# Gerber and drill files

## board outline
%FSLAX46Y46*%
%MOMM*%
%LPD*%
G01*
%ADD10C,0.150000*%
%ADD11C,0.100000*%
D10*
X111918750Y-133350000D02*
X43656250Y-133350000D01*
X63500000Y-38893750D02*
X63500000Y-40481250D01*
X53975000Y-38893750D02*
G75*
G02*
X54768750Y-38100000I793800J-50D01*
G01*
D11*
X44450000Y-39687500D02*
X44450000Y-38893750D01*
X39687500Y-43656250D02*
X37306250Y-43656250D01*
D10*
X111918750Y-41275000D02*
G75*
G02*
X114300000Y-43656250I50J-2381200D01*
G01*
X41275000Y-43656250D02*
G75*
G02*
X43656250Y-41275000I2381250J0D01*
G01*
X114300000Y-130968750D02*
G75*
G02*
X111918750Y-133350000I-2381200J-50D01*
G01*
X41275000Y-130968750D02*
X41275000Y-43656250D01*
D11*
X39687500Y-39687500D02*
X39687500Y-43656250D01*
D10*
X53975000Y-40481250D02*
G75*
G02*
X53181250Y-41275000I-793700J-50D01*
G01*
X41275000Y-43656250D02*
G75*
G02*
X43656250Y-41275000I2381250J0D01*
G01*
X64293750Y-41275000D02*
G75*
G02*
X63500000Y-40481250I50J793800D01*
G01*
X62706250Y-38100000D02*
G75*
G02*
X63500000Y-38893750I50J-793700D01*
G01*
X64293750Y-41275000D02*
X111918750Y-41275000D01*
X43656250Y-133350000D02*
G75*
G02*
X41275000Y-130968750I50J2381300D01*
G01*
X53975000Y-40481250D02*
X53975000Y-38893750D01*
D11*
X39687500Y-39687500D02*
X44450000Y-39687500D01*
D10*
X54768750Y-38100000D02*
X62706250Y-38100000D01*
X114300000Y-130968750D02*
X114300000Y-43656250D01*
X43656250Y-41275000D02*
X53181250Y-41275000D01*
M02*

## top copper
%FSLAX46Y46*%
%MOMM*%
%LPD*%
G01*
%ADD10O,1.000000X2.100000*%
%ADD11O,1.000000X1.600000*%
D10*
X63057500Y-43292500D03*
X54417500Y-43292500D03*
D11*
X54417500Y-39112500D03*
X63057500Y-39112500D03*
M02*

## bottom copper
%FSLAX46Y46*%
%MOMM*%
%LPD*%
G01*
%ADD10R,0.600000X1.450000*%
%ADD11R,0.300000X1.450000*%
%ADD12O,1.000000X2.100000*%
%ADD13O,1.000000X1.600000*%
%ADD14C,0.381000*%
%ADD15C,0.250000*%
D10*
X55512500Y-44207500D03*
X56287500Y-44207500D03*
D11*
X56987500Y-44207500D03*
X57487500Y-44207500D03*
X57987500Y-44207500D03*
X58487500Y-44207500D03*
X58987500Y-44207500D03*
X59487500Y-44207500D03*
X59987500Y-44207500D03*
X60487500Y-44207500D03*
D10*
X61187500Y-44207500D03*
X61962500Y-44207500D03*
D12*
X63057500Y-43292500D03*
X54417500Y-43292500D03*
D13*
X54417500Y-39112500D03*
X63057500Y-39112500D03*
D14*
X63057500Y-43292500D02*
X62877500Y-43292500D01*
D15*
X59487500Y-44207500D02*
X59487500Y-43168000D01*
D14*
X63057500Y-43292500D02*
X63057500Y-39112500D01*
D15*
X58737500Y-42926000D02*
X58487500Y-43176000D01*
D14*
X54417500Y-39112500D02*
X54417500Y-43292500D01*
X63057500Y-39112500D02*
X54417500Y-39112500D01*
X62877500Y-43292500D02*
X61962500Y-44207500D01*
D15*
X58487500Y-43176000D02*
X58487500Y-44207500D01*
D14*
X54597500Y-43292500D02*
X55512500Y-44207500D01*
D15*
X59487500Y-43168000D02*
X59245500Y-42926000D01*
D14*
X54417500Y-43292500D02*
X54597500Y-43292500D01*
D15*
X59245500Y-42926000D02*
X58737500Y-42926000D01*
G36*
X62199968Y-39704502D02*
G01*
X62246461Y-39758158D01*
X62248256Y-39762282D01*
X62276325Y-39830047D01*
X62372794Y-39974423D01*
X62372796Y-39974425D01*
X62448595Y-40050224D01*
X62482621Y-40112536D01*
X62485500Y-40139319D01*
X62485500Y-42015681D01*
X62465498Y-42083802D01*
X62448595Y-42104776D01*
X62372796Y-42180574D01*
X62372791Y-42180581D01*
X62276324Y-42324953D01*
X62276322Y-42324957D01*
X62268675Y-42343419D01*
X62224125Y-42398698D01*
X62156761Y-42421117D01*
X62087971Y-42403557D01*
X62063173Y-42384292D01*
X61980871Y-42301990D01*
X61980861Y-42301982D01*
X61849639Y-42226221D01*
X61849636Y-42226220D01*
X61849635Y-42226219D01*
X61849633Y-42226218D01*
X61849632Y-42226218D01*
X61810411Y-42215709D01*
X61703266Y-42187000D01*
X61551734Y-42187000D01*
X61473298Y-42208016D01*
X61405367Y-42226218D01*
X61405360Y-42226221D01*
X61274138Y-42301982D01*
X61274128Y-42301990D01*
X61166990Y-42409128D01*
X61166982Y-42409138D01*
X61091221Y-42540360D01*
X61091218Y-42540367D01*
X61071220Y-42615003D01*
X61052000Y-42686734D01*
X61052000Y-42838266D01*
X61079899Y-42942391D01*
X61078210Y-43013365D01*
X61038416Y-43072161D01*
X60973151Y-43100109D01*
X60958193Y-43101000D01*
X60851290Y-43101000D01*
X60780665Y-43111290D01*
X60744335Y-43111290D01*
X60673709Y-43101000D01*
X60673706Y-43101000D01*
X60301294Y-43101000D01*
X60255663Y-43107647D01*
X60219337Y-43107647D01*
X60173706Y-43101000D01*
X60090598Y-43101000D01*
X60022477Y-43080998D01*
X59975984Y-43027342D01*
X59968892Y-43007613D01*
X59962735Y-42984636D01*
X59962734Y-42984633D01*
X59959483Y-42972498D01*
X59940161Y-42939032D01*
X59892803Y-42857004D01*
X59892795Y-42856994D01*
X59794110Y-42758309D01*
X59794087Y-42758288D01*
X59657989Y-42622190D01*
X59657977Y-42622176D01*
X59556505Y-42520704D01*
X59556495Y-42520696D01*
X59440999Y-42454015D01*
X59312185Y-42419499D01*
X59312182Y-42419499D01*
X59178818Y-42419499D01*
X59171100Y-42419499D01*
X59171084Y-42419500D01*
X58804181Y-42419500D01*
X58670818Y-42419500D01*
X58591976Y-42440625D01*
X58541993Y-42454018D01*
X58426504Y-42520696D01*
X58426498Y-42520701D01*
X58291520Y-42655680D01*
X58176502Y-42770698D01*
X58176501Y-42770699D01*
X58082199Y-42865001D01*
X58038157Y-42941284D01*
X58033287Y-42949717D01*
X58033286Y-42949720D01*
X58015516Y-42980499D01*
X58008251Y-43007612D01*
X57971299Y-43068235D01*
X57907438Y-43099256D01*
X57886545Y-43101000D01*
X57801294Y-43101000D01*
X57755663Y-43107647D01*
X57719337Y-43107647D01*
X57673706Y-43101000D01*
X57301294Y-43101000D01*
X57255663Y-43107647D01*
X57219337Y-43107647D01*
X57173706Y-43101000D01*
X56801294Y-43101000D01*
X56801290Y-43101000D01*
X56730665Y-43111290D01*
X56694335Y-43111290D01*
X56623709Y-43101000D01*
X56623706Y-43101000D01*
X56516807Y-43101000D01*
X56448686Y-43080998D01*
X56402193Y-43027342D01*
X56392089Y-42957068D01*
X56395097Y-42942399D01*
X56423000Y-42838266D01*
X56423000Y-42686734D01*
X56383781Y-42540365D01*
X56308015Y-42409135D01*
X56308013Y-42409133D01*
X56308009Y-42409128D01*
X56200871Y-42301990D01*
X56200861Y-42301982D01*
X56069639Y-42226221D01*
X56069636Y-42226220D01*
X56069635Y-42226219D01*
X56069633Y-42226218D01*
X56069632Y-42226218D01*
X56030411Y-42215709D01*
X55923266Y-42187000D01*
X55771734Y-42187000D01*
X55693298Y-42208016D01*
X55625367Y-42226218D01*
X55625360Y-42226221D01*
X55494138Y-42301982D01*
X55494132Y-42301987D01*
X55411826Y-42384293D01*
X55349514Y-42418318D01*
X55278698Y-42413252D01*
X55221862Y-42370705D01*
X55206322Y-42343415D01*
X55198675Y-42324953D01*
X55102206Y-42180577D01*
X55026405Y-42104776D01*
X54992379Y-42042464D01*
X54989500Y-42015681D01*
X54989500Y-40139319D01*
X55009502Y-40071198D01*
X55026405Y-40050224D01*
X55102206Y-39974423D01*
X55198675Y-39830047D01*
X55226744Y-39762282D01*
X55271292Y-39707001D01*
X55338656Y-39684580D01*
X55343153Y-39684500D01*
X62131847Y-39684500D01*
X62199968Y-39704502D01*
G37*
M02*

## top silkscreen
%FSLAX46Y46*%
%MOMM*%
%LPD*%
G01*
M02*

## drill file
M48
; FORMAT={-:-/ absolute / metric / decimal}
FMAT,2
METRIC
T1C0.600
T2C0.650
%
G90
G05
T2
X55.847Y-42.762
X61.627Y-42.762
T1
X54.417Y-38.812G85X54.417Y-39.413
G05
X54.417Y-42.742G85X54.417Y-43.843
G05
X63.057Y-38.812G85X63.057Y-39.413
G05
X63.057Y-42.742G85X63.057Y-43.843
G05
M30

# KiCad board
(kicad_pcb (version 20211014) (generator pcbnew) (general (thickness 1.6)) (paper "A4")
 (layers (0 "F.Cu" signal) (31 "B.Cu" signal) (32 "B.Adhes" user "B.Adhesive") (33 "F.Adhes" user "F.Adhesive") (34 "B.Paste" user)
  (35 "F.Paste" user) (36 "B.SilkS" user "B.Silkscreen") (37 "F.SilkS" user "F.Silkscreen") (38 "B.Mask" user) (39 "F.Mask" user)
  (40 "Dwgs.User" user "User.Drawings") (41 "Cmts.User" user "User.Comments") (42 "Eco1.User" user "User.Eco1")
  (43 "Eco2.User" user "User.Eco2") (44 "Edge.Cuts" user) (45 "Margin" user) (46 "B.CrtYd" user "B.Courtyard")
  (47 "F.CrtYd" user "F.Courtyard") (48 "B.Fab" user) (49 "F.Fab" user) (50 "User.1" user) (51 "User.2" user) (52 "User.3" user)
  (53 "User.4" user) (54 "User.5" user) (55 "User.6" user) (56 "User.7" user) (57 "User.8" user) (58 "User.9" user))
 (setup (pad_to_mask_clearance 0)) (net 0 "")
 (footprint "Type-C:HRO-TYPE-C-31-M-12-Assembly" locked (layer "B.Cu") (at 58.7375 36.5125)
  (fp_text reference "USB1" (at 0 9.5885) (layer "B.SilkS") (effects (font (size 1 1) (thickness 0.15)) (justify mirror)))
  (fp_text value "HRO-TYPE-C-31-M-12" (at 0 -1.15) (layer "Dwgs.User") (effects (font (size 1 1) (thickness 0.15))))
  (pad "" np_thru_hole circle locked (at -2.89 6.25) (size 0.65 0.65) (drill 0.65) (layers *.Cu *.Mask))
  (pad "" np_thru_hole circle locked (at 2.89 6.25) (size 0.65 0.65) (drill 0.65) (layers *.Cu *.Mask))
  (pad "1" smd rect locked (at -3.225 7.695) (size 0.6 1.45) (layers "B.Cu" "B.Paste" "B.Mask"))
  (pad "2" smd rect locked (at -2.45 7.695) (size 0.6 1.45) (layers "B.Cu" "B.Paste" "B.Mask"))
  (pad "3" smd rect locked (at -1.75 7.695) (size 0.3 1.45) (layers "B.Cu" "B.Paste" "B.Mask"))
  (pad "4" smd rect locked (at -1.25 7.695) (size 0.3 1.45) (layers "B.Cu" "B.Paste" "B.Mask"))
  (pad "5" smd rect locked (at -0.75 7.695) (size 0.3 1.45) (layers "B.Cu" "B.Paste" "B.Mask"))
  (pad "6" smd rect locked (at -0.25 7.695) (size 0.3 1.45) (layers "B.Cu" "B.Paste" "B.Mask"))
  (pad "7" smd rect locked (at 0.25 7.695) (size 0.3 1.45) (layers "B.Cu" "B.Paste" "B.Mask"))
  (pad "8" smd rect locked (at 0.75 7.695) (size 0.3 1.45) (layers "B.Cu" "B.Paste" "B.Mask"))
  (pad "9" smd rect locked (at 1.25 7.695) (size 0.3 1.45) (layers "B.Cu" "B.Paste" "B.Mask"))
  (pad "10" smd rect locked (at 1.75 7.695) (size 0.3 1.45) (layers "B.Cu" "B.Paste" "B.Mask"))
  (pad "11" smd rect locked (at 2.45 7.695) (size 0.6 1.45) (layers "B.Cu" "B.Paste" "B.Mask"))
  (pad "12" smd rect locked (at 3.225 7.695) (size 0.6 1.45) (layers "B.Cu" "B.Paste" "B.Mask"))
  (pad "13" thru_hole oval locked (at 4.32 6.78) (size 1 2.1) (drill oval 0.6 1.7) (layers *.Cu *.Mask))
  (pad "13" thru_hole oval locked (at -4.32 6.78) (size 1 2.1) (drill oval 0.6 1.7) (layers *.Cu *.Mask))
  (pad "13" thru_hole oval locked (at -4.32 2.6) (size 1 1.6) (drill oval 0.6 1.2) (layers *.Cu *.Mask))
  (pad "13" thru_hole oval locked (at 4.32 2.6) (size 1 1.6) (drill oval 0.6 1.2) (layers *.Cu *.Mask)))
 (gr_line locked (start 111.91875 133.35) (end 43.65625 133.35) (layer "Edge.Cuts") (width 0.15))
 (gr_line locked (start 63.5 38.89375) (end 63.5 40.48125) (layer "Edge.Cuts") (width 0.15))
 (gr_arc locked (start 53.975 38.89375) (mid 54.207485 38.332485) (end 54.76875 38.1) (layer "Edge.Cuts") (width 0.15))
 (gr_line locked (start 44.45 39.6875) (end 44.45 38.89375) (layer "Edge.Cuts") (width 0.1))
 (gr_line locked (start 39.6875 43.65625) (end 37.30625 43.65625) (layer "Edge.Cuts") (width 0.1))
 (gr_arc locked (start 111.91875 41.275) (mid 113.60255 41.972451) (end 114.3 43.65625) (layer "Edge.Cuts") (width 0.15))
 (gr_arc locked (start 41.275 43.65625) (mid 41.972452 41.972452) (end 43.65625 41.275) (layer "Edge.Cuts") (width 0.15))
 (gr_arc locked (start 114.3 130.96875) (mid 113.602549 132.652549) (end 111.91875 133.35) (layer "Edge.Cuts") (width 0.15))
 (gr_line locked (start 41.275 130.96875) (end 41.275 43.65625) (layer "Edge.Cuts") (width 0.15))
 (gr_line locked (start 39.6875 39.6875) (end 39.6875 43.65625) (layer "Edge.Cuts") (width 0.1))
 (gr_arc locked (start 53.975 40.48125) (mid 53.742517 41.042517) (end 53.18125 41.275) (layer "Edge.Cuts") (width 0.15))
 (gr_arc locked (start 41.275 43.65625) (mid 41.972452 41.972452) (end 43.65625 41.275) (layer "Edge.Cuts") (width 0.15))
 (gr_arc locked (start 64.29375 41.275) (mid 63.732486 41.042515) (end 63.5 40.48125) (layer "Edge.Cuts") (width 0.15))
 (gr_arc locked (start 62.70625 38.1) (mid 63.267518 38.332483) (end 63.5 38.89375) (layer "Edge.Cuts") (width 0.15))
 (gr_line locked (start 64.29375 41.275) (end 111.91875 41.275) (layer "Edge.Cuts") (width 0.15))
 (gr_arc locked (start 43.65625 133.35) (mid 41.972454 132.652547) (end 41.275 130.96875) (layer "Edge.Cuts") (width 0.15))
 (gr_line locked (start 53.975 40.48125) (end 53.975 38.89375) (layer "Edge.Cuts") (width 0.15))
 (gr_line locked (start 39.6875 39.6875) (end 44.45 39.6875) (layer "Edge.Cuts") (width 0.1))
 (gr_line locked (start 54.76875 38.1) (end 62.70625 38.1) (layer "Edge.Cuts") (width 0.15))
 (gr_line locked (start 114.3 130.96875) (end 114.3 43.65625) (layer "Edge.Cuts") (width 0.15))
 (gr_line locked (start 43.65625 41.275) (end 53.18125 41.275) (layer "Edge.Cuts") (width 0.15))
 (segment (start 63.0575 43.2925) (end 62.8775 43.2925) (width 0.381) (layer "B.Cu") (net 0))
 (segment (start 59.4875 44.2075) (end 59.4875 43.168) (width 0.25) (layer "B.Cu") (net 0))
 (segment (start 63.0575 43.2925) (end 63.0575 39.1125) (width 0.381) (layer "B.Cu") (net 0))
 (segment (start 58.7375 42.926) (end 58.4875 43.176) (width 0.25) (layer "B.Cu") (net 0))
 (segment (start 54.4175 39.1125) (end 54.4175 43.2925) (width 0.381) (layer "B.Cu") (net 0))
 (segment (start 63.0575 39.1125) (end 54.4175 39.1125) (width 0.381) (layer "B.Cu") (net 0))
 (segment (start 62.8775 43.2925) (end 61.9625 44.2075) (width 0.381) (layer "B.Cu") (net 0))
 (segment (start 58.4875 43.176) (end 58.4875 44.2075) (width 0.25) (layer "B.Cu") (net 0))
 (segment (start 54.5975 43.2925) (end 55.5125 44.2075) (width 0.381) (layer "B.Cu") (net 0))
 (segment (start 59.4875 43.168) (end 59.2455 42.926) (width 0.25) (layer "B.Cu") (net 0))
 (segment (start 54.4175 43.2925) (end 54.5975 43.2925) (width 0.381) (layer "B.Cu") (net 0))
 (segment (start 59.2455 42.926) (end 58.7375 42.926) (width 0.25) (layer "B.Cu") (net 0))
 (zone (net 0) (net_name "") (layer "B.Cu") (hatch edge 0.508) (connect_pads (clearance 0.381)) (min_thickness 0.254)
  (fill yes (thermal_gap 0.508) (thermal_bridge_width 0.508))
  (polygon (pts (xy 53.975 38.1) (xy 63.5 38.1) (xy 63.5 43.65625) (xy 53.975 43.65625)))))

